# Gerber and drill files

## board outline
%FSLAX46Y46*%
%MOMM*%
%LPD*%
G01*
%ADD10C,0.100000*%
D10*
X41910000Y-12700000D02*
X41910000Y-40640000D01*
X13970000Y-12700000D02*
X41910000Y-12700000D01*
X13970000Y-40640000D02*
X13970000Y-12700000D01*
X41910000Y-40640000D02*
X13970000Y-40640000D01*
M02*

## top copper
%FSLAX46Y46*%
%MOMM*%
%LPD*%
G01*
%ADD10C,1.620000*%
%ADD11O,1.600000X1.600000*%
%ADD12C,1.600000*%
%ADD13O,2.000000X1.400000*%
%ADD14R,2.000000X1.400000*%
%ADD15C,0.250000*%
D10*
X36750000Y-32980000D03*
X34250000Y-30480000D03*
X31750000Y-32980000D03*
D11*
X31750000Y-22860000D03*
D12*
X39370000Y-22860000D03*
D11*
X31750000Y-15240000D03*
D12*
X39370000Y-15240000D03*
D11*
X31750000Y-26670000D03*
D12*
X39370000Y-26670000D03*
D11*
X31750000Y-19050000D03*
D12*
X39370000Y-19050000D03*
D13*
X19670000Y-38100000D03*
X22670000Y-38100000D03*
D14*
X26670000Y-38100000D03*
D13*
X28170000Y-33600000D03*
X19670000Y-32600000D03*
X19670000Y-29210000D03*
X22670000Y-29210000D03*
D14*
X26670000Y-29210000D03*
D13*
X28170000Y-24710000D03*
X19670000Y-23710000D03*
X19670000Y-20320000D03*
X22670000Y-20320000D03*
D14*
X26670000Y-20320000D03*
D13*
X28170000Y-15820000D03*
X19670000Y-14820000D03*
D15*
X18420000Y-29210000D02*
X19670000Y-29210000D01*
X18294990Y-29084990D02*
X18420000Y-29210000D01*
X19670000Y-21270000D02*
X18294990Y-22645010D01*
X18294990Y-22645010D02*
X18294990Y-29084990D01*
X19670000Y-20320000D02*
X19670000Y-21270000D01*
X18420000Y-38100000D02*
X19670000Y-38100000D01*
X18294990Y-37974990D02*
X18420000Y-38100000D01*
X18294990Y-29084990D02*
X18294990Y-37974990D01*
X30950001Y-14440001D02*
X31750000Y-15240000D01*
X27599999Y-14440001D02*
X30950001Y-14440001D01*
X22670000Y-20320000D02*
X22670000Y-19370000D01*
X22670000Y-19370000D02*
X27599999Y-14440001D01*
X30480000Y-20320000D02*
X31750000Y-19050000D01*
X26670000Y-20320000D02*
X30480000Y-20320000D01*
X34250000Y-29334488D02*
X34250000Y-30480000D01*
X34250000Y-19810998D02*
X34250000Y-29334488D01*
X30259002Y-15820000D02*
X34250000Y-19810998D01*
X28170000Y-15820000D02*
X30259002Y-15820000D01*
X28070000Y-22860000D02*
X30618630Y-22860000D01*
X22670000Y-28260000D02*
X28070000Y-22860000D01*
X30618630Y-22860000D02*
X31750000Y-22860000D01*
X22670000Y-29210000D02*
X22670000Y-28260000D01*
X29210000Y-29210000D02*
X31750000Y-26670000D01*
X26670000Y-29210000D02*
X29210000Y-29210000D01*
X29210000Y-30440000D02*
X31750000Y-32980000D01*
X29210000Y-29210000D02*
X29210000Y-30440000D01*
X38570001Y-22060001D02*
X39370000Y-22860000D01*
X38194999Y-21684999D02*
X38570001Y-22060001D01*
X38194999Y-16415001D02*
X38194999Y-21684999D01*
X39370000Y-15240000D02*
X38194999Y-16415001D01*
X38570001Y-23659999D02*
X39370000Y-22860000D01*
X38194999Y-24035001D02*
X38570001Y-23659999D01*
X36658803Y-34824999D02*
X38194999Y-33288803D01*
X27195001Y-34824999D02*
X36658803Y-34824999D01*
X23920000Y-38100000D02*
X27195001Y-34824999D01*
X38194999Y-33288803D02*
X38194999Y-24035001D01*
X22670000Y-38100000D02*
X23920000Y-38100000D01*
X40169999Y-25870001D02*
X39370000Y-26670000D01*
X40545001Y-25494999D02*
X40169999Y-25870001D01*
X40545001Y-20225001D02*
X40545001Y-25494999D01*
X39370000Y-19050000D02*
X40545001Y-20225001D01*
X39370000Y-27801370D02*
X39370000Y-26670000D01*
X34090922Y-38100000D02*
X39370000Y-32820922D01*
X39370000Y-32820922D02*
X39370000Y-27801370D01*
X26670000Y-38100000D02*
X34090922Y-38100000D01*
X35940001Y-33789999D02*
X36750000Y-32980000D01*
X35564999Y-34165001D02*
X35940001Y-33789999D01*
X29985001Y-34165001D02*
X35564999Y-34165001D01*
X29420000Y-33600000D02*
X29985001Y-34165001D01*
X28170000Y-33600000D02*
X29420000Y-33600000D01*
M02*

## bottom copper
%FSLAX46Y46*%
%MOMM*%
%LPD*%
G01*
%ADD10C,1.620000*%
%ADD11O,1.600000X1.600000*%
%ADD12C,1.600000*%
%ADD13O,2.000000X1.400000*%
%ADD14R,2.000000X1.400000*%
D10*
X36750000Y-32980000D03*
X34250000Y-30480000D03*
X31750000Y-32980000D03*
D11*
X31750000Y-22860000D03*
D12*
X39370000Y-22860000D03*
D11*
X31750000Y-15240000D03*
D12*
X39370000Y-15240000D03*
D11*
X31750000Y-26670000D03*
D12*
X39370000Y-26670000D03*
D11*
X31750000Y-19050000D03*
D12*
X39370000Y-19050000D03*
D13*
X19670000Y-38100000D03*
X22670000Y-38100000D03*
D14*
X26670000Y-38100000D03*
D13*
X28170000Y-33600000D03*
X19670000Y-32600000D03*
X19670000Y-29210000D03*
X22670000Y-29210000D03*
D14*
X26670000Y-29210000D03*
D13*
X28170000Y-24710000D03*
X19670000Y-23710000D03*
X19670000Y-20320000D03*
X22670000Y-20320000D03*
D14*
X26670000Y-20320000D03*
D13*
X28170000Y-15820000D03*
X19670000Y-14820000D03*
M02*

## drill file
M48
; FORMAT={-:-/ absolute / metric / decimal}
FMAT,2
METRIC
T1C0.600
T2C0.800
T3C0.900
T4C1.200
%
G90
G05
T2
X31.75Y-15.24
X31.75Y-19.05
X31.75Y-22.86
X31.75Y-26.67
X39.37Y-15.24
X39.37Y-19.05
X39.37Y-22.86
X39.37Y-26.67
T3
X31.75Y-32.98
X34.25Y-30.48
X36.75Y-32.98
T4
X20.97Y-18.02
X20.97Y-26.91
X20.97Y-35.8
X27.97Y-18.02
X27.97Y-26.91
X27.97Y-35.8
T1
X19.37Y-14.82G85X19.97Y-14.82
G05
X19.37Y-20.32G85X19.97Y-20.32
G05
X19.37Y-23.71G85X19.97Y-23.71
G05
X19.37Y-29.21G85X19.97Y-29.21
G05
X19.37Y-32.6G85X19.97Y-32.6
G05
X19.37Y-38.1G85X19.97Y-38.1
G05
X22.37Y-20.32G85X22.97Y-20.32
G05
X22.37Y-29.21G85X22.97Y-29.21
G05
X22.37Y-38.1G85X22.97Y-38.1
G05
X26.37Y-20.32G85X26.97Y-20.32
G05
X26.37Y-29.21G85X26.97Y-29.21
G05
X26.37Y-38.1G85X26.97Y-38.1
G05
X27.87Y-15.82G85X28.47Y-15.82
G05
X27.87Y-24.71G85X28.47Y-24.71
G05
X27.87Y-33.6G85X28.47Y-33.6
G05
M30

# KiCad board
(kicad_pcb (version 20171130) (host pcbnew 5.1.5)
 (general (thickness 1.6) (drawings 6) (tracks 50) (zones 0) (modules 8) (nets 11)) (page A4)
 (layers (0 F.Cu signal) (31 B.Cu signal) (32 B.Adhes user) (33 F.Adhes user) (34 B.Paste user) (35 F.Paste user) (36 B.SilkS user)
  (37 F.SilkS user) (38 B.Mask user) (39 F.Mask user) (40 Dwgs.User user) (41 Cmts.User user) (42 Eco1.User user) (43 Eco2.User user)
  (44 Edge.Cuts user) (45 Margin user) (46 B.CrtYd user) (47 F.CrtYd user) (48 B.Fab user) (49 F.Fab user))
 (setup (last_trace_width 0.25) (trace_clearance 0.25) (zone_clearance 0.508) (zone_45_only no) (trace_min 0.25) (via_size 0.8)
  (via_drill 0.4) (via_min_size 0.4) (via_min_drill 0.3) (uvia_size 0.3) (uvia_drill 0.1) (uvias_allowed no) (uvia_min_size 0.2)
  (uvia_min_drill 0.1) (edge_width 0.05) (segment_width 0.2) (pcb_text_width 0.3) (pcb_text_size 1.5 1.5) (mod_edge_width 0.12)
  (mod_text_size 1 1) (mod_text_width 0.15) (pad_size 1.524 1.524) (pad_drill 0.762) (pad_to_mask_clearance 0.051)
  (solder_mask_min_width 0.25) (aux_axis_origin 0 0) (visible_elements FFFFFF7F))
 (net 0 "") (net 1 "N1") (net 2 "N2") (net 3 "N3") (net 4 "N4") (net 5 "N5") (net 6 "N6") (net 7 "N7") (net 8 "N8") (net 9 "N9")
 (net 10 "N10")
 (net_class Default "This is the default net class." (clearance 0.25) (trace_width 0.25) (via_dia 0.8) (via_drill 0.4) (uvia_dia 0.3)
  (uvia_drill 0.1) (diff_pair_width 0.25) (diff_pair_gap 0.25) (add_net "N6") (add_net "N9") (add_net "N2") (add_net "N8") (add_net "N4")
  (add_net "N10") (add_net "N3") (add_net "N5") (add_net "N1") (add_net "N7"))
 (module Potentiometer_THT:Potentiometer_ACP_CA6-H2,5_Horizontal (layer F.Cu) (at 31.75 32.98 90)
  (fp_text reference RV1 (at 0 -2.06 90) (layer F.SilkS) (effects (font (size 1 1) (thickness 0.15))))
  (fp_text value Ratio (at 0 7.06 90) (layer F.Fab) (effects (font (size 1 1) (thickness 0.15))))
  (pad 3 thru_hole circle (at 0 5 90) (size 1.62 1.62) (drill 0.9) (layers *.Cu *.Mask) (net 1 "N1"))
  (pad 2 thru_hole circle (at 2.5 2.5 90) (size 1.62 1.62) (drill 0.9) (layers *.Cu *.Mask) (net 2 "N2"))
  (pad 1 thru_hole circle (at 0 0 90) (size 1.62 1.62) (drill 0.9) (layers *.Cu *.Mask) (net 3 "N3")))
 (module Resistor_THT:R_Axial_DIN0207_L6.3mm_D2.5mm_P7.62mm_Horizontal (layer F.Cu) (at 39.37 22.86 180)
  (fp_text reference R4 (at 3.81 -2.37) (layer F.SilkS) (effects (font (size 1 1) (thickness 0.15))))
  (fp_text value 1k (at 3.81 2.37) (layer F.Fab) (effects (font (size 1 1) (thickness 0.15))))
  (pad 2 thru_hole oval (at 7.62 0 180) (size 1.6 1.6) (drill 0.8) (layers *.Cu *.Mask) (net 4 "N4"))
  (pad 1 thru_hole circle (at 0 0 180) (size 1.6 1.6) (drill 0.8) (layers *.Cu *.Mask) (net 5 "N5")))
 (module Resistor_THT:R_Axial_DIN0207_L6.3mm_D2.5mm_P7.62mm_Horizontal (layer F.Cu) (at 39.37 15.24 180)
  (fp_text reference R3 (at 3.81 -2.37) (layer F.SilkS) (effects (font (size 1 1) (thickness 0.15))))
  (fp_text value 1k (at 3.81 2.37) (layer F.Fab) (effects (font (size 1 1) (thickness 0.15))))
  (pad 2 thru_hole oval (at 7.62 0 180) (size 1.6 1.6) (drill 0.8) (layers *.Cu *.Mask) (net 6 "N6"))
  (pad 1 thru_hole circle (at 0 0 180) (size 1.6 1.6) (drill 0.8) (layers *.Cu *.Mask) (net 5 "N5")))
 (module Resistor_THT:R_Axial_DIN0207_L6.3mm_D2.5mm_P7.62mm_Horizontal (layer F.Cu) (at 39.37 26.67 180)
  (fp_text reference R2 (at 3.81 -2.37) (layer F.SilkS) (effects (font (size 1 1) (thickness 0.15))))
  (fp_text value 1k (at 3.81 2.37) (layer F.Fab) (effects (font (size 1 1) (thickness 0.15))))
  (pad 2 thru_hole oval (at 7.62 0 180) (size 1.6 1.6) (drill 0.8) (layers *.Cu *.Mask) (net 3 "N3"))
  (pad 1 thru_hole circle (at 0 0 180) (size 1.6 1.6) (drill 0.8) (layers *.Cu *.Mask) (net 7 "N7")))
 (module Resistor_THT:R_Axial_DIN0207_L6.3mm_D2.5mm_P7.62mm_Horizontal (layer F.Cu) (at 39.37 19.05 180)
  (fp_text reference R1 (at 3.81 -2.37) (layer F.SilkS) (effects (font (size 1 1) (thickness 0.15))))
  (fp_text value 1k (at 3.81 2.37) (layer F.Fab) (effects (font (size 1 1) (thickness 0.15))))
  (pad 2 thru_hole oval (at 7.62 0 180) (size 1.6 1.6) (drill 0.8) (layers *.Cu *.Mask) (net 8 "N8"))
  (pad 1 thru_hole circle (at 0 0 180) (size 1.6 1.6) (drill 0.8) (layers *.Cu *.Mask) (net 7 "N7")))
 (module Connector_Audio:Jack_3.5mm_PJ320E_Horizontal (layer F.Cu) (at 26.67 38.1 90)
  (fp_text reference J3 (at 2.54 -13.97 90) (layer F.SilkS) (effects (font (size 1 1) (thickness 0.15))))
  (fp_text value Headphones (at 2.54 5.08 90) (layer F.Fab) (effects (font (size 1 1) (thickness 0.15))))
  (pad "" np_thru_hole circle (at 2.3 1.3) (size 1.2 1.2) (drill 1.2) (layers *.Cu *.Mask))
  (pad "" np_thru_hole circle (at 2.3 -5.7) (size 1.2 1.2) (drill 1.2) (layers *.Cu *.Mask))
  (pad R2 thru_hole oval (at 0 -7) (size 2 1.4) (drill oval 1.2 0.6) (layers *.Cu *.Mask) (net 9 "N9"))
  (pad R1 thru_hole oval (at 0 -4) (size 2 1.4) (drill oval 1.2 0.6) (layers *.Cu *.Mask) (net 5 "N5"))
  (pad T thru_hole rect (at 0 0) (size 2 1.4) (drill oval 1.2 0.6) (layers *.Cu *.Mask) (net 7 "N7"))
  (pad S thru_hole oval (at 4.5 1.5) (size 2 1.4) (drill oval 1.2 0.6) (layers *.Cu *.Mask) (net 1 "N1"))
  (pad "" thru_hole oval (at 5.5 -7) (size 2 1.4) (drill oval 1.2 0.6) (layers *.Cu *.Mask)))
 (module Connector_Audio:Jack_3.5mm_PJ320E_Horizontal (layer F.Cu) (at 26.67 29.21 90)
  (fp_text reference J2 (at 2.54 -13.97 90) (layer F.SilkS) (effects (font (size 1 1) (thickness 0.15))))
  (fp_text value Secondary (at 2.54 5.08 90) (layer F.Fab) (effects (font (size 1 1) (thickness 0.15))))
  (pad "" np_thru_hole circle (at 2.3 1.3) (size 1.2 1.2) (drill 1.2) (layers *.Cu *.Mask))
  (pad "" np_thru_hole circle (at 2.3 -5.7) (size 1.2 1.2) (drill 1.2) (layers *.Cu *.Mask))
  (pad R2 thru_hole oval (at 0 -7) (size 2 1.4) (drill oval 1.2 0.6) (layers *.Cu *.Mask) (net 9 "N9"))
  (pad R1 thru_hole oval (at 0 -4) (size 2 1.4) (drill oval 1.2 0.6) (layers *.Cu *.Mask) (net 4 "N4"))
  (pad T thru_hole rect (at 0 0) (size 2 1.4) (drill oval 1.2 0.6) (layers *.Cu *.Mask) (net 3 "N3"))
  (pad S thru_hole oval (at 4.5 1.5) (size 2 1.4) (drill oval 1.2 0.6) (layers *.Cu *.Mask) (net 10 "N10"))
  (pad "" thru_hole oval (at 5.5 -7) (size 2 1.4) (drill oval 1.2 0.6) (layers *.Cu *.Mask)))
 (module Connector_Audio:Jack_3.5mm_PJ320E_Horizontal (layer F.Cu) (at 26.67 20.32 90)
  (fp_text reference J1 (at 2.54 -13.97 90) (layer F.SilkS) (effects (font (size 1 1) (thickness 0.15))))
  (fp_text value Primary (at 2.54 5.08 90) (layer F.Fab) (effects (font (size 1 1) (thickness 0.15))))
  (pad "" np_thru_hole circle (at 2.3 1.3) (size 1.2 1.2) (drill 1.2) (layers *.Cu *.Mask))
  (pad "" np_thru_hole circle (at 2.3 -5.7) (size 1.2 1.2) (drill 1.2) (layers *.Cu *.Mask))
  (pad R2 thru_hole oval (at 0 -7) (size 2 1.4) (drill oval 1.2 0.6) (layers *.Cu *.Mask) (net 9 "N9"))
  (pad R1 thru_hole oval (at 0 -4) (size 2 1.4) (drill oval 1.2 0.6) (layers *.Cu *.Mask) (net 6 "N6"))
  (pad T thru_hole rect (at 0 0) (size 2 1.4) (drill oval 1.2 0.6) (layers *.Cu *.Mask) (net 8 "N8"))
  (pad S thru_hole oval (at 4.5 1.5) (size 2 1.4) (drill oval 1.2 0.6) (layers *.Cu *.Mask) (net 2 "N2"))
  (pad "" thru_hole oval (at 5.5 -7) (size 2 1.4) (drill oval 1.2 0.6) (layers *.Cu *.Mask)))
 (gr_line (start 41.91 12.7) (end 41.91 40.64) (layer Edge.Cuts) (width 0.1))
 (gr_line (start 13.97 12.7) (end 41.91 12.7) (layer Edge.Cuts) (width 0.1))
 (gr_line (start 13.97 40.64) (end 13.97 12.7) (layer Edge.Cuts) (width 0.1))
 (gr_line (start 41.91 40.64) (end 13.97 40.64) (layer Edge.Cuts) (width 0.1))
 (segment (start 18.42 29.21) (end 19.67 29.21) (width 0.25) (layer F.Cu) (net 9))
 (segment (start 18.29499 29.08499) (end 18.42 29.21) (width 0.25) (layer F.Cu) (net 9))
 (segment (start 19.67 21.27) (end 18.29499 22.64501) (width 0.25) (layer F.Cu) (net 9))
 (segment (start 18.29499 22.64501) (end 18.29499 29.08499) (width 0.25) (layer F.Cu) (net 9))
 (segment (start 19.67 20.32) (end 19.67 21.27) (width 0.25) (layer F.Cu) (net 9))
 (segment (start 18.42 38.1) (end 19.67 38.1) (width 0.25) (layer F.Cu) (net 9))
 (segment (start 18.29499 37.97499) (end 18.42 38.1) (width 0.25) (layer F.Cu) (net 9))
 (segment (start 18.29499 29.08499) (end 18.29499 37.97499) (width 0.25) (layer F.Cu) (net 9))
 (segment (start 30.950001 14.440001) (end 31.75 15.24) (width 0.25) (layer F.Cu) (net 6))
 (segment (start 27.599999 14.440001) (end 30.950001 14.440001) (width 0.25) (layer F.Cu) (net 6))
 (segment (start 22.67 20.32) (end 22.67 19.37) (width 0.25) (layer F.Cu) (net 6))
 (segment (start 22.67 19.37) (end 27.599999 14.440001) (width 0.25) (layer F.Cu) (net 6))
 (segment (start 30.48 20.32) (end 31.75 19.05) (width 0.25) (layer F.Cu) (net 8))
 (segment (start 26.67 20.32) (end 30.48 20.32) (width 0.25) (layer F.Cu) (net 8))
 (segment (start 34.25 29.334488) (end 34.25 30.48) (width 0.25) (layer F.Cu) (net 2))
 (segment (start 34.25 19.810998) (end 34.25 29.334488) (width 0.25) (layer F.Cu) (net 2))
 (segment (start 30.259002 15.82) (end 34.25 19.810998) (width 0.25) (layer F.Cu) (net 2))
 (segment (start 28.17 15.82) (end 30.259002 15.82) (width 0.25) (layer F.Cu) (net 2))
 (segment (start 28.07 22.86) (end 30.61863 22.86) (width 0.25) (layer F.Cu) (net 4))
 (segment (start 22.67 28.26) (end 28.07 22.86) (width 0.25) (layer F.Cu) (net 4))
 (segment (start 30.61863 22.86) (end 31.75 22.86) (width 0.25) (layer F.Cu) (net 4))
 (segment (start 22.67 29.21) (end 22.67 28.26) (width 0.25) (layer F.Cu) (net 4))
 (segment (start 29.21 29.21) (end 31.75 26.67) (width 0.25) (layer F.Cu) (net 3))
 (segment (start 26.67 29.21) (end 29.21 29.21) (width 0.25) (layer F.Cu) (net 3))
 (segment (start 29.21 30.44) (end 31.75 32.98) (width 0.25) (layer F.Cu) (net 3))
 (segment (start 29.21 29.21) (end 29.21 30.44) (width 0.25) (layer F.Cu) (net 3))
 (segment (start 38.570001 22.060001) (end 39.37 22.86) (width 0.25) (layer F.Cu) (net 5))
 (segment (start 38.194999 21.684999) (end 38.570001 22.060001) (width 0.25) (layer F.Cu) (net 5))
 (segment (start 38.194999 16.415001) (end 38.194999 21.684999) (width 0.25) (layer F.Cu) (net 5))
 (segment (start 39.37 15.24) (end 38.194999 16.415001) (width 0.25) (layer F.Cu) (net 5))
 (segment (start 38.570001 23.659999) (end 39.37 22.86) (width 0.25) (layer F.Cu) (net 5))
 (segment (start 38.194999 24.035001) (end 38.570001 23.659999) (width 0.25) (layer F.Cu) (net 5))
 (segment (start 36.658803 34.824999) (end 38.194999 33.288803) (width 0.25) (layer F.Cu) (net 5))
 (segment (start 27.195001 34.824999) (end 36.658803 34.824999) (width 0.25) (layer F.Cu) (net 5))
 (segment (start 23.92 38.1) (end 27.195001 34.824999) (width 0.25) (layer F.Cu) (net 5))
 (segment (start 38.194999 33.288803) (end 38.194999 24.035001) (width 0.25) (layer F.Cu) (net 5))
 (segment (start 22.67 38.1) (end 23.92 38.1) (width 0.25) (layer F.Cu) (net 5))
 (segment (start 40.169999 25.870001) (end 39.37 26.67) (width 0.25) (layer F.Cu) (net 7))
 (segment (start 40.545001 25.494999) (end 40.169999 25.870001) (width 0.25) (layer F.Cu) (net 7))
 (segment (start 40.545001 20.225001) (end 40.545001 25.494999) (width 0.25) (layer F.Cu) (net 7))
 (segment (start 39.37 19.05) (end 40.545001 20.225001) (width 0.25) (layer F.Cu) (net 7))
 (segment (start 39.37 27.80137) (end 39.37 26.67) (width 0.25) (layer F.Cu) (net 7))
 (segment (start 34.090922 38.1) (end 39.37 32.820922) (width 0.25) (layer F.Cu) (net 7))
 (segment (start 39.37 32.820922) (end 39.37 27.80137) (width 0.25) (layer F.Cu) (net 7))
 (segment (start 26.67 38.1) (end 34.090922 38.1) (width 0.25) (layer F.Cu) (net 7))
 (segment (start 35.940001 33.789999) (end 36.75 32.98) (width 0.25) (layer F.Cu) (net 1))
 (segment (start 35.564999 34.165001) (end 35.940001 33.789999) (width 0.25) (layer F.Cu) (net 1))
 (segment (start 29.985001 34.165001) (end 35.564999 34.165001) (width 0.25) (layer F.Cu) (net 1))
 (segment (start 29.42 33.6) (end 29.985001 34.165001) (width 0.25) (layer F.Cu) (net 1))
 (segment (start 28.17 33.6) (end 29.42 33.6) (width 0.25) (layer F.Cu) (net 1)))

